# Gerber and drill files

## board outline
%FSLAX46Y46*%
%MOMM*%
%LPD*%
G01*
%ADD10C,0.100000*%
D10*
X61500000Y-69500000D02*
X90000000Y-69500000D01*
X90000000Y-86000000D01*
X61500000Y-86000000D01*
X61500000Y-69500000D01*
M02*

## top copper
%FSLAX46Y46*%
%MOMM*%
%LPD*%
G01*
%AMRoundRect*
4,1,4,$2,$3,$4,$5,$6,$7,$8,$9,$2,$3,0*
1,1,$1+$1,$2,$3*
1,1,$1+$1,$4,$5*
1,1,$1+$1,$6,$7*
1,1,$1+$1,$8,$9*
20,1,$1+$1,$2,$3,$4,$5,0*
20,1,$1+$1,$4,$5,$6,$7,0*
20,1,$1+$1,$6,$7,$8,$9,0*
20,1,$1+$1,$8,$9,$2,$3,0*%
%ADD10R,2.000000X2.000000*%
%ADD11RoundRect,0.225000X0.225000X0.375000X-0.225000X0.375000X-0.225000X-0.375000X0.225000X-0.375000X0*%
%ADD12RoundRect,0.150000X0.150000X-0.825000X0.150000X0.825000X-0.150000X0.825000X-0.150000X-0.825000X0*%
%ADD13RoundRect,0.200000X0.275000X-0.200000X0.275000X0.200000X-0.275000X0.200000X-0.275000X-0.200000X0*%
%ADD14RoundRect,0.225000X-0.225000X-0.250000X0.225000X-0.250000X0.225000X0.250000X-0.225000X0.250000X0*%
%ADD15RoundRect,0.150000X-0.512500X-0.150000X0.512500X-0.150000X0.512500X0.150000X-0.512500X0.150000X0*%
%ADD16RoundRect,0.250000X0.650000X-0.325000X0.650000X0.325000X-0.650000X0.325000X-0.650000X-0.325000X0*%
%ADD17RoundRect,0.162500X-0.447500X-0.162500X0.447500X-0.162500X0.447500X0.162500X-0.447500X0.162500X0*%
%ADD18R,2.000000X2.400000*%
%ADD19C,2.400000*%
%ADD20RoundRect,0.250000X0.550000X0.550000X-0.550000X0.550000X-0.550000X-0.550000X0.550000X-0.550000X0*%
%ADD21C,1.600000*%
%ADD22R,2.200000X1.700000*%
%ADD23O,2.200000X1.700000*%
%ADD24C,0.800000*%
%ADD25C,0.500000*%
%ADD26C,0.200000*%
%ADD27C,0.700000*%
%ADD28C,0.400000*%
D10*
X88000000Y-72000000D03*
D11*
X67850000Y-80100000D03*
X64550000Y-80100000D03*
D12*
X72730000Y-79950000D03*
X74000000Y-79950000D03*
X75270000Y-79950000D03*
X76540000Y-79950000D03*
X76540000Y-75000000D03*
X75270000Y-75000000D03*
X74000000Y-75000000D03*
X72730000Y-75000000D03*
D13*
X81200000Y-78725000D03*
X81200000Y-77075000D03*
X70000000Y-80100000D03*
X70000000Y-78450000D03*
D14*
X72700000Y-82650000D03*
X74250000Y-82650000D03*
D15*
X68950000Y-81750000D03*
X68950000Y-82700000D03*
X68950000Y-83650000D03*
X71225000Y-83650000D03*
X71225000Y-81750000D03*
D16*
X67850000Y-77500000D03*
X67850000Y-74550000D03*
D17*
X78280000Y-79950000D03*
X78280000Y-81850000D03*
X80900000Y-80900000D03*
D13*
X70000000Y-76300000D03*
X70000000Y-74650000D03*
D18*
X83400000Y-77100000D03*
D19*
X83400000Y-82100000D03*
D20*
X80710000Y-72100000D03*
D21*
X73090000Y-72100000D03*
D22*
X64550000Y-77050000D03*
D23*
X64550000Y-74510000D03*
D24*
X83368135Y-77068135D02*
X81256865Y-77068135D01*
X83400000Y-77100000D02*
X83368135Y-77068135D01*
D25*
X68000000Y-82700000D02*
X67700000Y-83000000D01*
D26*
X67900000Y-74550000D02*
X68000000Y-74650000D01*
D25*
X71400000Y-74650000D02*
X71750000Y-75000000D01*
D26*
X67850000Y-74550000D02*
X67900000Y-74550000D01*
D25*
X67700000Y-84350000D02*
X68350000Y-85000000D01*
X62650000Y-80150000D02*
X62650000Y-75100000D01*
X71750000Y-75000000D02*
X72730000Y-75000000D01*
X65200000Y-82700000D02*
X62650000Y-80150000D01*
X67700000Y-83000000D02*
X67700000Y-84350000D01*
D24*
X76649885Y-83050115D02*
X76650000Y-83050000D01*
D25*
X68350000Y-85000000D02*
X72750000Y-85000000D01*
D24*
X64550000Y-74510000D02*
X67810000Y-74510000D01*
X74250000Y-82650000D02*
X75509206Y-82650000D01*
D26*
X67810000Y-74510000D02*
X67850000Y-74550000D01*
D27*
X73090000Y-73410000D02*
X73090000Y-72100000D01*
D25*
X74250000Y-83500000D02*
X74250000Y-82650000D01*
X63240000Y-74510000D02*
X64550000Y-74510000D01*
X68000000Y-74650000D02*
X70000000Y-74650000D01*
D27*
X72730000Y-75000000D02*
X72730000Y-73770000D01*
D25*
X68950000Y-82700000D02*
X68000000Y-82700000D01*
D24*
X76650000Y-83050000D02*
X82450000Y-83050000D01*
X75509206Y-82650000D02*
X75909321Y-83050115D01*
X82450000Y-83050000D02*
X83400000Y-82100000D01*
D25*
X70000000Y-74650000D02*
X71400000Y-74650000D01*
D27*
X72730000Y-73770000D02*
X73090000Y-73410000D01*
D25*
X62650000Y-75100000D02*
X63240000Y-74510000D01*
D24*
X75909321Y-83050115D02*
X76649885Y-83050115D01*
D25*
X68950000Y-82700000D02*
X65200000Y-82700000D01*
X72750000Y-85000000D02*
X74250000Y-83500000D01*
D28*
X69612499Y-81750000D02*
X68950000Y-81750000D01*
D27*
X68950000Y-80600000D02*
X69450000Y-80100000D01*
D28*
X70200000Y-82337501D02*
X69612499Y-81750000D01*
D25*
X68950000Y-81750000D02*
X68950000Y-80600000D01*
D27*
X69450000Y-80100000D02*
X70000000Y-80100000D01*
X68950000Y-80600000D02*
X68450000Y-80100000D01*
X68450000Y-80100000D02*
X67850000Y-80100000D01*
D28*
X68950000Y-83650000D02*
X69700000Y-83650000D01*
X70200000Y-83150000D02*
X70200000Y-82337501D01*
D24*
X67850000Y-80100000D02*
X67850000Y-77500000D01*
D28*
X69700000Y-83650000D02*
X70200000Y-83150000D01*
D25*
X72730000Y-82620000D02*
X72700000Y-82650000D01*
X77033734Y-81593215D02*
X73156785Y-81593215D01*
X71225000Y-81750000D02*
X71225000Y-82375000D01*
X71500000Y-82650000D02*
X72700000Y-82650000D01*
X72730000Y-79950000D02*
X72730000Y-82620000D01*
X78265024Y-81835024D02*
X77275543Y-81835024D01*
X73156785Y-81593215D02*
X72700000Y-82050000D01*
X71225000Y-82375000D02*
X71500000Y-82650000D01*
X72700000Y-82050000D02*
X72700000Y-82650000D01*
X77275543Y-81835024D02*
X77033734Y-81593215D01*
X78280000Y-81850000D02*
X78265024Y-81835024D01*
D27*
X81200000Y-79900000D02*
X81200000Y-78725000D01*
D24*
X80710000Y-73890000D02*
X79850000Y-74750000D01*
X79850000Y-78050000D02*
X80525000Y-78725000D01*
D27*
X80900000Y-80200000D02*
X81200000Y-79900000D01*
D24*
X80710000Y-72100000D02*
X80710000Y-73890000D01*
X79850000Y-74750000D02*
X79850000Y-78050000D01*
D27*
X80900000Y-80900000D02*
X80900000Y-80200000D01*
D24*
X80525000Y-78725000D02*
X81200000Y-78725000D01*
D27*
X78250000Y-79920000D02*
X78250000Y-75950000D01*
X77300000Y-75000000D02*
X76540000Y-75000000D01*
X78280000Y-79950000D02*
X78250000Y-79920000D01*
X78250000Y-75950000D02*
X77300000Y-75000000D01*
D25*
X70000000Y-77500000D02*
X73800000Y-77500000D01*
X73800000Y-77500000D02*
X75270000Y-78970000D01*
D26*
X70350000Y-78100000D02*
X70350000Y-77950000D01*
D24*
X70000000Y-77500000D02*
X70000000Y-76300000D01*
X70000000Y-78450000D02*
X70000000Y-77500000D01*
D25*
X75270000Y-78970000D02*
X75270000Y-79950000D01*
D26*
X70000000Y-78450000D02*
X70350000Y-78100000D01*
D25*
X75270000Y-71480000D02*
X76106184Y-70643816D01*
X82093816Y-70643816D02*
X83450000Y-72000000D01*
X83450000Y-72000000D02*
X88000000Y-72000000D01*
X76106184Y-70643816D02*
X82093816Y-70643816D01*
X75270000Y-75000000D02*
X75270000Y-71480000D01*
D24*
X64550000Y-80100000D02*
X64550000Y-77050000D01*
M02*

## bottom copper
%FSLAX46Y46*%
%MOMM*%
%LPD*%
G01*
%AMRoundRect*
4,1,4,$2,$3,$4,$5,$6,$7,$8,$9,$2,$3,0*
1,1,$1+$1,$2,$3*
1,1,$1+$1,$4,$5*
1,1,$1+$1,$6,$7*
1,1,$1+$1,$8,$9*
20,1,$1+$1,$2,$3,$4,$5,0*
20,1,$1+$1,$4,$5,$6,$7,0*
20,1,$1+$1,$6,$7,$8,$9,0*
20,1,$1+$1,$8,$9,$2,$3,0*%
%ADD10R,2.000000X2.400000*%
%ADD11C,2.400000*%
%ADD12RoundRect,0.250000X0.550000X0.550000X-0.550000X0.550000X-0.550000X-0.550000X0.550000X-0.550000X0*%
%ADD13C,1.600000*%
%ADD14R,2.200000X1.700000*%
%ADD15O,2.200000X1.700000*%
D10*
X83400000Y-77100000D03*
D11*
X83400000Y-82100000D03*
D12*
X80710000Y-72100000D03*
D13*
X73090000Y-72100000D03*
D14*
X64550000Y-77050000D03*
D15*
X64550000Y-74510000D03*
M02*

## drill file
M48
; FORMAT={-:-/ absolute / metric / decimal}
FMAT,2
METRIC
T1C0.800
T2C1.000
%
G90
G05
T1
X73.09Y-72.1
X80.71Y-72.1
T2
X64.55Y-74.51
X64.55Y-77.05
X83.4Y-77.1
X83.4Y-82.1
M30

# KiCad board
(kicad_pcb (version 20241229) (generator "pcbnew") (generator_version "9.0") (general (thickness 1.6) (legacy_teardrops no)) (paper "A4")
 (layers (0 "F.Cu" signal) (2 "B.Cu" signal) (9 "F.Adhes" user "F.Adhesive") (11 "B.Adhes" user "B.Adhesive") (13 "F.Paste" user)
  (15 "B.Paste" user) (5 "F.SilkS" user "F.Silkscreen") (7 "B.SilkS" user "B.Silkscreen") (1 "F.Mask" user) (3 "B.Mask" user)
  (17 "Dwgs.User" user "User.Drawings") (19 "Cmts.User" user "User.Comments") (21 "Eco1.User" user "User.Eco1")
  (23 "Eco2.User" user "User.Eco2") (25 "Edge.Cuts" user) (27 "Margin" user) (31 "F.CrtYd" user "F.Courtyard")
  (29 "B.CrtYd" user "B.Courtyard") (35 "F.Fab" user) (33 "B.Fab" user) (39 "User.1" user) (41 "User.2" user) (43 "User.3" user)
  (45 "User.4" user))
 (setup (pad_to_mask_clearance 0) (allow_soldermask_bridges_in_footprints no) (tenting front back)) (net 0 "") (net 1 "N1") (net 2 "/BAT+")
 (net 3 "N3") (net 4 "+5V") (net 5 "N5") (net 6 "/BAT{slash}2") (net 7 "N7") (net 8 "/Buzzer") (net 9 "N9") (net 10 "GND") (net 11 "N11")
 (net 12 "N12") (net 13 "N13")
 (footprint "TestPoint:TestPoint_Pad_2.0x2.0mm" (layer "F.Cu") (at 88 72)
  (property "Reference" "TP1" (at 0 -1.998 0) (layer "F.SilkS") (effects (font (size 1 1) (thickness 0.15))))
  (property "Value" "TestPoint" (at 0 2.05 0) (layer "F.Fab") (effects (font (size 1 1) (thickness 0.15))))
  (pad "1" smd rect (at 0 0) (size 2 2) (layers "F.Cu" "F.Mask") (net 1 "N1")))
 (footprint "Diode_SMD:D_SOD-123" (layer "F.Cu") (at 66.2 80.1 180)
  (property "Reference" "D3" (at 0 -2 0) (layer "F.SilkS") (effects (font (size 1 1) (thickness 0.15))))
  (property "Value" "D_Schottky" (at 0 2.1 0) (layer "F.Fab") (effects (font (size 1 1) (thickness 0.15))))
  (pad "1" smd roundrect (at -1.65 0 180) (size 0.9 1.2) (layers "F.Cu" "F.Mask" "F.Paste") (roundrect_rratio 0.25) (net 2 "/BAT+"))
  (pad "2" smd roundrect (at 1.65 0 180) (size 0.9 1.2) (layers "F.Cu" "F.Mask" "F.Paste") (roundrect_rratio 0.25) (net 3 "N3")))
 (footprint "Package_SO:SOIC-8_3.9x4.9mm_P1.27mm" (layer "F.Cu") (at 74.635 77.475 90)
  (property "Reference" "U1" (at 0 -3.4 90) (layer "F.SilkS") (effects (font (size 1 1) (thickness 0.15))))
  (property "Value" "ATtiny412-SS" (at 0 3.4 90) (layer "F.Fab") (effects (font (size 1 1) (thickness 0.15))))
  (pad "1" smd roundrect (at -2.475 -1.905 90) (size 1.95 0.6) (layers "F.Cu" "F.Mask" "F.Paste") (roundrect_rratio 0.25) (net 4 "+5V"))
  (pad "2" smd roundrect (at -2.475 -0.635 90) (size 1.95 0.6) (layers "F.Cu" "F.Mask" "F.Paste") (roundrect_rratio 0.25) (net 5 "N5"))
  (pad "3" smd roundrect (at -2.475 0.635 90) (size 1.95 0.6) (layers "F.Cu" "F.Mask" "F.Paste") (roundrect_rratio 0.25)
   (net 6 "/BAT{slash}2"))
  (pad "4" smd roundrect (at -2.475 1.905 90) (size 1.95 0.6) (layers "F.Cu" "F.Mask" "F.Paste") (roundrect_rratio 0.25) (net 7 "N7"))
  (pad "5" smd roundrect (at 2.475 1.905 90) (size 1.95 0.6) (layers "F.Cu" "F.Mask" "F.Paste") (roundrect_rratio 0.25) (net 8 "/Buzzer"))
  (pad "6" smd roundrect (at 2.475 0.635 90) (size 1.95 0.6) (layers "F.Cu" "F.Mask" "F.Paste") (roundrect_rratio 0.25) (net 1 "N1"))
  (pad "7" smd roundrect (at 2.475 -0.635 90) (size 1.95 0.6) (layers "F.Cu" "F.Mask" "F.Paste") (roundrect_rratio 0.25) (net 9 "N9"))
  (pad "8" smd roundrect (at 2.475 -1.905 90) (size 1.95 0.6) (layers "F.Cu" "F.Mask" "F.Paste") (roundrect_rratio 0.25) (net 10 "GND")))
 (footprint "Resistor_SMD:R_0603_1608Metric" (layer "F.Cu") (at 81.2 77.9 90)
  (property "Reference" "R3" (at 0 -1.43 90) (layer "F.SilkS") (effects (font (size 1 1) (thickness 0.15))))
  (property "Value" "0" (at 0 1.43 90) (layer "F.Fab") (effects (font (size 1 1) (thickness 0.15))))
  (pad "1" smd roundrect (at -0.825 0 90) (size 0.8 0.95) (layers "F.Cu" "F.Mask" "F.Paste") (roundrect_rratio 0.25) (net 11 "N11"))
  (pad "2" smd roundrect (at 0.825 0 90) (size 0.8 0.95) (layers "F.Cu" "F.Mask" "F.Paste") (roundrect_rratio 0.25) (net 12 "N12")))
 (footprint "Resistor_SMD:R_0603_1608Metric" (layer "F.Cu") (at 70 79.275 90)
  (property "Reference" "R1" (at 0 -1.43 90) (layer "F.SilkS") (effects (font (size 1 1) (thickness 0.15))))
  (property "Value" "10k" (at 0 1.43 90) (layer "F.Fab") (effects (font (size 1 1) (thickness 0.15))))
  (pad "1" smd roundrect (at -0.825 0 90) (size 0.8 0.95) (layers "F.Cu" "F.Mask" "F.Paste") (roundrect_rratio 0.25) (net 2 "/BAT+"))
  (pad "2" smd roundrect (at 0.825 0 90) (size 0.8 0.95) (layers "F.Cu" "F.Mask" "F.Paste") (roundrect_rratio 0.25) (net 6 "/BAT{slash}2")))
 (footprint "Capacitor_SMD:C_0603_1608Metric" (layer "F.Cu") (at 73.475 82.65)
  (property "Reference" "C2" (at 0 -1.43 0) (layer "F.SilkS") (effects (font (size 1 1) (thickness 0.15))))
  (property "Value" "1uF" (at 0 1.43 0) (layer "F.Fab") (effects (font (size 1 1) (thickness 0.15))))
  (pad "1" smd roundrect (at -0.775 0) (size 0.9 0.95) (layers "F.Cu" "F.Mask" "F.Paste") (roundrect_rratio 0.25) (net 4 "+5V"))
  (pad "2" smd roundrect (at 0.775 0) (size 0.9 0.95) (layers "F.Cu" "F.Mask" "F.Paste") (roundrect_rratio 0.25) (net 10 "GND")))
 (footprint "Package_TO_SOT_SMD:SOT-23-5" (layer "F.Cu") (at 70.0875 82.7)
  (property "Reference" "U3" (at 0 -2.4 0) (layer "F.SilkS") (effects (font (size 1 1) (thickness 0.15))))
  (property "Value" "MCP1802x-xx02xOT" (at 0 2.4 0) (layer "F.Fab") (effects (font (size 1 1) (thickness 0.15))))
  (pad "1" smd roundrect (at -1.1375 -0.95) (size 1.325 0.6) (layers "F.Cu" "F.Mask" "F.Paste") (roundrect_rratio 0.25) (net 2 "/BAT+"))
  (pad "2" smd roundrect (at -1.1375 0) (size 1.325 0.6) (layers "F.Cu" "F.Mask" "F.Paste") (roundrect_rratio 0.25) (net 10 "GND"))
  (pad "3" smd roundrect (at -1.1375 0.95) (size 1.325 0.6) (layers "F.Cu" "F.Mask" "F.Paste") (roundrect_rratio 0.25) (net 2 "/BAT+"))
  (pad "4" smd roundrect (at 1.1375 0.95) (size 1.325 0.6) (layers "F.Cu" "F.Mask" "F.Paste") (roundrect_rratio 0.25) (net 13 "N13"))
  (pad "5" smd roundrect (at 1.1375 -0.95) (size 1.325 0.6) (layers "F.Cu" "F.Mask" "F.Paste") (roundrect_rratio 0.25) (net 4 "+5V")))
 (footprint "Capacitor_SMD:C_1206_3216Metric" (layer "F.Cu") (at 67.85 76.025 90)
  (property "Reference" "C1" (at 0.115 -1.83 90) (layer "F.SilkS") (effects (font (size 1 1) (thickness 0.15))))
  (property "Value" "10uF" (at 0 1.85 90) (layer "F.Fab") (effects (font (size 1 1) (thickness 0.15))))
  (pad "1" smd roundrect (at -1.475 0 90) (size 1.15 1.8) (layers "F.Cu" "F.Mask" "F.Paste") (roundrect_rratio 0.217391) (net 2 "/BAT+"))
  (pad "2" smd roundrect (at 1.475 0 90) (size 1.15 1.8) (layers "F.Cu" "F.Mask" "F.Paste") (roundrect_rratio 0.217391) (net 10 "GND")))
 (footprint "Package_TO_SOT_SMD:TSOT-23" (layer "F.Cu") (at 79.59 80.9)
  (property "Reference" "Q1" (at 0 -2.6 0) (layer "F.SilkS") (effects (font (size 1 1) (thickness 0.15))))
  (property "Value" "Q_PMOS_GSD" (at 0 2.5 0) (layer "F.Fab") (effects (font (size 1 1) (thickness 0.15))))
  (pad "1" smd roundrect (at -1.31 -0.95) (size 1.22 0.65) (layers "F.Cu" "F.Mask" "F.Paste") (roundrect_rratio 0.25) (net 8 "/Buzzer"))
  (pad "2" smd roundrect (at -1.31 0.95) (size 1.22 0.65) (layers "F.Cu" "F.Mask" "F.Paste") (roundrect_rratio 0.25) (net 4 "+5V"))
  (pad "3" smd roundrect (at 1.31 0) (size 1.22 0.65) (layers "F.Cu" "F.Mask" "F.Paste") (roundrect_rratio 0.25) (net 11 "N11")))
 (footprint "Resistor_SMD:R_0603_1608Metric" (layer "F.Cu") (at 70 75.475 90)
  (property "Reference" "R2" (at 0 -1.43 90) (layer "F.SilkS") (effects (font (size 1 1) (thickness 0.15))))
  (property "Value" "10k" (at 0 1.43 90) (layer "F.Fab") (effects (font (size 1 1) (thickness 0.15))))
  (pad "1" smd roundrect (at -0.825 0 90) (size 0.8 0.95) (layers "F.Cu" "F.Mask" "F.Paste") (roundrect_rratio 0.25) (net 6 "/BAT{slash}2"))
  (pad "2" smd roundrect (at 0.825 0 90) (size 0.8 0.95) (layers "F.Cu" "F.Mask" "F.Paste") (roundrect_rratio 0.25) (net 10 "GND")))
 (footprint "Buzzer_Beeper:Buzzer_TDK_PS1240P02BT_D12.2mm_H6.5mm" (layer "B.Cu") (at 83.4 77.1 -90)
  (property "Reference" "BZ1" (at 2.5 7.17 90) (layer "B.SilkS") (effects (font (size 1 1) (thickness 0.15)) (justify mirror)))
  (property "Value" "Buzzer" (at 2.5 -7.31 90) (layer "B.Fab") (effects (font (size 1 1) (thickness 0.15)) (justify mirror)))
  (pad "1" thru_hole rect (at 0 0 270) (size 2.4 2) (drill 1) (layers "*.Cu" "*.Mask") (remove_unused_layers no) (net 12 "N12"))
  (pad "2" thru_hole circle (at 5 0 270) (size 2.4 2.4) (drill 1) (layers "*.Cu" "*.Mask") (remove_unused_layers no) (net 10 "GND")))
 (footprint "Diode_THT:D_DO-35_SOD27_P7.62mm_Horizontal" (layer "B.Cu") (at 80.71 72.1 180)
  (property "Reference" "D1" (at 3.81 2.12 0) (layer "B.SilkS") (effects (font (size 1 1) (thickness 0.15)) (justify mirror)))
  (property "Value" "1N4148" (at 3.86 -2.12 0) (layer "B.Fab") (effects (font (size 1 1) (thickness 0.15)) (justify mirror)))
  (pad "1" thru_hole roundrect (at 0 0 180) (size 1.6 1.6) (drill 0.8) (layers "*.Cu" "*.Mask") (remove_unused_layers no)
   (roundrect_rratio 0.15625) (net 11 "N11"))
  (pad "2" thru_hole circle (at 7.62 0 180) (size 1.6 1.6) (drill 0.8) (layers "*.Cu" "*.Mask") (remove_unused_layers no) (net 10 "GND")))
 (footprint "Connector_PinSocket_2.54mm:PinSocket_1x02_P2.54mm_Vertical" (layer "B.Cu") (at 64.55 77.05)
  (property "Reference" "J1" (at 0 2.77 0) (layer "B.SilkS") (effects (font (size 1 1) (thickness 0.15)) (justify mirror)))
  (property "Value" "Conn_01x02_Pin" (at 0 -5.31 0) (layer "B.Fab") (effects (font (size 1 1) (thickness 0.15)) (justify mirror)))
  (pad "1" thru_hole rect (at 0 0) (size 2.2 1.7) (drill 1) (layers "*.Cu" "*.Mask") (remove_unused_layers no) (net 3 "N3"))
  (pad "2" thru_hole oval (at 0 -2.54) (size 2.2 1.7) (drill 1) (layers "*.Cu" "*.Mask") (remove_unused_layers no) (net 10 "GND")))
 (gr_rect (start 61.5 69.5) (end 90 86) (stroke (width 0.1) (type solid)) (fill no) (layer "Edge.Cuts"))
 (segment (start 83.368135 77.068135) (end 81.256865 77.068135) (width 0.8) (layer "F.Cu") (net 12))
 (segment (start 83.4 77.1) (end 83.368135 77.068135) (width 0.8) (layer "F.Cu") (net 12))
 (segment (start 68 82.7) (end 67.7 83) (width 0.5) (layer "F.Cu") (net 10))
 (segment (start 67.9 74.55) (end 68 74.65) (width 0.2) (layer "F.Cu") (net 10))
 (segment (start 71.4 74.65) (end 71.75 75) (width 0.5) (layer "F.Cu") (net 10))
 (segment (start 67.85 74.55) (end 67.9 74.55) (width 0.2) (layer "F.Cu") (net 10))
 (segment (start 67.7 84.35) (end 68.35 85) (width 0.5) (layer "F.Cu") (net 10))
 (segment (start 62.65 80.15) (end 62.65 75.1) (width 0.5) (layer "F.Cu") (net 10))
 (segment (start 71.75 75) (end 72.73 75) (width 0.5) (layer "F.Cu") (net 10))
 (segment (start 65.2 82.7) (end 62.65 80.15) (width 0.5) (layer "F.Cu") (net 10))
 (segment (start 67.7 83) (end 67.7 84.35) (width 0.5) (layer "F.Cu") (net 10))
 (segment (start 76.649885 83.050115) (end 76.65 83.05) (width 0.8) (layer "F.Cu") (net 10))
 (segment (start 68.35 85) (end 72.75 85) (width 0.5) (layer "F.Cu") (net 10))
 (segment (start 64.55 74.51) (end 67.81 74.51) (width 0.8) (layer "F.Cu") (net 10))
 (segment (start 74.25 82.65) (end 75.509206 82.65) (width 0.8) (layer "F.Cu") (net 10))
 (segment (start 67.81 74.51) (end 67.85 74.55) (width 0.2) (layer "F.Cu") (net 10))
 (segment (start 73.09 73.41) (end 73.09 72.1) (width 0.7) (layer "F.Cu") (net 10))
 (segment (start 74.25 83.5) (end 74.25 82.65) (width 0.5) (layer "F.Cu") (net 10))
 (segment (start 63.24 74.51) (end 64.55 74.51) (width 0.5) (layer "F.Cu") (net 10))
 (segment (start 68 74.65) (end 70 74.65) (width 0.5) (layer "F.Cu") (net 10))
 (segment (start 72.73 75) (end 72.73 73.77) (width 0.7) (layer "F.Cu") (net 10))
 (segment (start 68.95 82.7) (end 68 82.7) (width 0.5) (layer "F.Cu") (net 10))
 (segment (start 76.65 83.05) (end 82.45 83.05) (width 0.8) (layer "F.Cu") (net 10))
 (segment (start 75.509206 82.65) (end 75.909321 83.050115) (width 0.8) (layer "F.Cu") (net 10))
 (segment (start 82.45 83.05) (end 83.4 82.1) (width 0.8) (layer "F.Cu") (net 10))
 (segment (start 70 74.65) (end 71.4 74.65) (width 0.5) (layer "F.Cu") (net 10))
 (segment (start 72.73 73.77) (end 73.09 73.41) (width 0.7) (layer "F.Cu") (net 10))
 (segment (start 62.65 75.1) (end 63.24 74.51) (width 0.5) (layer "F.Cu") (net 10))
 (segment (start 75.909321 83.050115) (end 76.649885 83.050115) (width 0.8) (layer "F.Cu") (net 10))
 (segment (start 68.95 82.7) (end 65.2 82.7) (width 0.5) (layer "F.Cu") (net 10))
 (segment (start 72.75 85) (end 74.25 83.5) (width 0.5) (layer "F.Cu") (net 10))
 (segment (start 69.612499 81.75) (end 68.95 81.75) (width 0.4) (layer "F.Cu") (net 2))
 (segment (start 68.95 80.6) (end 69.45 80.1) (width 0.7) (layer "F.Cu") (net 2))
 (segment (start 70.2 82.337501) (end 69.612499 81.75) (width 0.4) (layer "F.Cu") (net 2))
 (segment (start 68.95 81.75) (end 68.95 80.6) (width 0.5) (layer "F.Cu") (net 2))
 (segment (start 69.45 80.1) (end 70 80.1) (width 0.7) (layer "F.Cu") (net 2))
 (segment (start 68.95 80.6) (end 68.45 80.1) (width 0.7) (layer "F.Cu") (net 2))
 (segment (start 68.45 80.1) (end 67.85 80.1) (width 0.7) (layer "F.Cu") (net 2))
 (segment (start 68.95 83.65) (end 69.7 83.65) (width 0.4) (layer "F.Cu") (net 2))
 (segment (start 70.2 83.15) (end 70.2 82.337501) (width 0.4) (layer "F.Cu") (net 2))
 (segment (start 67.85 80.1) (end 67.85 77.5) (width 0.8) (layer "F.Cu") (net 2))
 (segment (start 69.7 83.65) (end 70.2 83.15) (width 0.4) (layer "F.Cu") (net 2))
 (segment (start 72.73 82.62) (end 72.7 82.65) (width 0.5) (layer "F.Cu") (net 4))
 (segment (start 77.033734 81.593215) (end 73.156785 81.593215) (width 0.5) (layer "F.Cu") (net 4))
 (segment (start 71.225 81.75) (end 71.225 82.375) (width 0.5) (layer "F.Cu") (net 4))
 (segment (start 71.5 82.65) (end 72.7 82.65) (width 0.5) (layer "F.Cu") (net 4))
 (segment (start 72.73 79.95) (end 72.73 82.62) (width 0.5) (layer "F.Cu") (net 4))
 (segment (start 78.265024 81.835024) (end 77.275543 81.835024) (width 0.5) (layer "F.Cu") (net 4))
 (segment (start 73.156785 81.593215) (end 72.7 82.05) (width 0.5) (layer "F.Cu") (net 4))
 (segment (start 71.225 82.375) (end 71.5 82.65) (width 0.5) (layer "F.Cu") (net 4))
 (segment (start 72.7 82.05) (end 72.7 82.65) (width 0.5) (layer "F.Cu") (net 4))
 (segment (start 77.275543 81.835024) (end 77.033734 81.593215) (width 0.5) (layer "F.Cu") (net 4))
 (segment (start 78.28 81.85) (end 78.265024 81.835024) (width 0.5) (layer "F.Cu") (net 4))
 (segment (start 81.2 79.9) (end 81.2 78.725) (width 0.7) (layer "F.Cu") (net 11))
 (segment (start 80.71 73.89) (end 79.85 74.75) (width 0.8) (layer "F.Cu") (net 11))
 (segment (start 79.85 78.05) (end 80.525 78.725) (width 0.8) (layer "F.Cu") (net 11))
 (segment (start 80.9 80.2) (end 81.2 79.9) (width 0.7) (layer "F.Cu") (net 11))
 (segment (start 80.71 72.1) (end 80.71 73.89) (width 0.8) (layer "F.Cu") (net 11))
 (segment (start 79.85 74.75) (end 79.85 78.05) (width 0.8) (layer "F.Cu") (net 11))
 (segment (start 80.9 80.9) (end 80.9 80.2) (width 0.7) (layer "F.Cu") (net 11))
 (segment (start 80.525 78.725) (end 81.2 78.725) (width 0.8) (layer "F.Cu") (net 11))
 (segment (start 78.25 79.92) (end 78.25 75.95) (width 0.7) (layer "F.Cu") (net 8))
 (segment (start 77.3 75) (end 76.54 75) (width 0.7) (layer "F.Cu") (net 8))
 (segment (start 78.28 79.95) (end 78.25 79.92) (width 0.7) (layer "F.Cu") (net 8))
 (segment (start 78.25 75.95) (end 77.3 75) (width 0.7) (layer "F.Cu") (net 8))
 (segment (start 70 77.5) (end 73.8 77.5) (width 0.5) (layer "F.Cu") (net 6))
 (segment (start 73.8 77.5) (end 75.27 78.97) (width 0.5) (layer "F.Cu") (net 6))
 (segment (start 70.35 78.1) (end 70.35 77.95) (width 0.2) (layer "F.Cu") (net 6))
 (segment (start 70 77.5) (end 70 76.3) (width 0.8) (layer "F.Cu") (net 6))
 (segment (start 70 78.45) (end 70 77.5) (width 0.8) (layer "F.Cu") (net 6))
 (segment (start 75.27 78.97) (end 75.27 79.95) (width 0.5) (layer "F.Cu") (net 6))
 (segment (start 70 78.45) (end 70.35 78.1) (width 0.2) (layer "F.Cu") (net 6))
 (segment (start 75.27 71.48) (end 76.106184 70.643816) (width 0.5) (layer "F.Cu") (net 1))
 (segment (start 82.093816 70.643816) (end 83.45 72) (width 0.5) (layer "F.Cu") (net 1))
 (segment (start 83.45 72) (end 88 72) (width 0.5) (layer "F.Cu") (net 1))
 (segment (start 76.106184 70.643816) (end 82.093816 70.643816) (width 0.5) (layer "F.Cu") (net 1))
 (segment (start 75.27 75) (end 75.27 71.48) (width 0.5) (layer "F.Cu") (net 1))
 (segment (start 64.55 80.1) (end 64.55 77.05) (width 0.8) (layer "F.Cu") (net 3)))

